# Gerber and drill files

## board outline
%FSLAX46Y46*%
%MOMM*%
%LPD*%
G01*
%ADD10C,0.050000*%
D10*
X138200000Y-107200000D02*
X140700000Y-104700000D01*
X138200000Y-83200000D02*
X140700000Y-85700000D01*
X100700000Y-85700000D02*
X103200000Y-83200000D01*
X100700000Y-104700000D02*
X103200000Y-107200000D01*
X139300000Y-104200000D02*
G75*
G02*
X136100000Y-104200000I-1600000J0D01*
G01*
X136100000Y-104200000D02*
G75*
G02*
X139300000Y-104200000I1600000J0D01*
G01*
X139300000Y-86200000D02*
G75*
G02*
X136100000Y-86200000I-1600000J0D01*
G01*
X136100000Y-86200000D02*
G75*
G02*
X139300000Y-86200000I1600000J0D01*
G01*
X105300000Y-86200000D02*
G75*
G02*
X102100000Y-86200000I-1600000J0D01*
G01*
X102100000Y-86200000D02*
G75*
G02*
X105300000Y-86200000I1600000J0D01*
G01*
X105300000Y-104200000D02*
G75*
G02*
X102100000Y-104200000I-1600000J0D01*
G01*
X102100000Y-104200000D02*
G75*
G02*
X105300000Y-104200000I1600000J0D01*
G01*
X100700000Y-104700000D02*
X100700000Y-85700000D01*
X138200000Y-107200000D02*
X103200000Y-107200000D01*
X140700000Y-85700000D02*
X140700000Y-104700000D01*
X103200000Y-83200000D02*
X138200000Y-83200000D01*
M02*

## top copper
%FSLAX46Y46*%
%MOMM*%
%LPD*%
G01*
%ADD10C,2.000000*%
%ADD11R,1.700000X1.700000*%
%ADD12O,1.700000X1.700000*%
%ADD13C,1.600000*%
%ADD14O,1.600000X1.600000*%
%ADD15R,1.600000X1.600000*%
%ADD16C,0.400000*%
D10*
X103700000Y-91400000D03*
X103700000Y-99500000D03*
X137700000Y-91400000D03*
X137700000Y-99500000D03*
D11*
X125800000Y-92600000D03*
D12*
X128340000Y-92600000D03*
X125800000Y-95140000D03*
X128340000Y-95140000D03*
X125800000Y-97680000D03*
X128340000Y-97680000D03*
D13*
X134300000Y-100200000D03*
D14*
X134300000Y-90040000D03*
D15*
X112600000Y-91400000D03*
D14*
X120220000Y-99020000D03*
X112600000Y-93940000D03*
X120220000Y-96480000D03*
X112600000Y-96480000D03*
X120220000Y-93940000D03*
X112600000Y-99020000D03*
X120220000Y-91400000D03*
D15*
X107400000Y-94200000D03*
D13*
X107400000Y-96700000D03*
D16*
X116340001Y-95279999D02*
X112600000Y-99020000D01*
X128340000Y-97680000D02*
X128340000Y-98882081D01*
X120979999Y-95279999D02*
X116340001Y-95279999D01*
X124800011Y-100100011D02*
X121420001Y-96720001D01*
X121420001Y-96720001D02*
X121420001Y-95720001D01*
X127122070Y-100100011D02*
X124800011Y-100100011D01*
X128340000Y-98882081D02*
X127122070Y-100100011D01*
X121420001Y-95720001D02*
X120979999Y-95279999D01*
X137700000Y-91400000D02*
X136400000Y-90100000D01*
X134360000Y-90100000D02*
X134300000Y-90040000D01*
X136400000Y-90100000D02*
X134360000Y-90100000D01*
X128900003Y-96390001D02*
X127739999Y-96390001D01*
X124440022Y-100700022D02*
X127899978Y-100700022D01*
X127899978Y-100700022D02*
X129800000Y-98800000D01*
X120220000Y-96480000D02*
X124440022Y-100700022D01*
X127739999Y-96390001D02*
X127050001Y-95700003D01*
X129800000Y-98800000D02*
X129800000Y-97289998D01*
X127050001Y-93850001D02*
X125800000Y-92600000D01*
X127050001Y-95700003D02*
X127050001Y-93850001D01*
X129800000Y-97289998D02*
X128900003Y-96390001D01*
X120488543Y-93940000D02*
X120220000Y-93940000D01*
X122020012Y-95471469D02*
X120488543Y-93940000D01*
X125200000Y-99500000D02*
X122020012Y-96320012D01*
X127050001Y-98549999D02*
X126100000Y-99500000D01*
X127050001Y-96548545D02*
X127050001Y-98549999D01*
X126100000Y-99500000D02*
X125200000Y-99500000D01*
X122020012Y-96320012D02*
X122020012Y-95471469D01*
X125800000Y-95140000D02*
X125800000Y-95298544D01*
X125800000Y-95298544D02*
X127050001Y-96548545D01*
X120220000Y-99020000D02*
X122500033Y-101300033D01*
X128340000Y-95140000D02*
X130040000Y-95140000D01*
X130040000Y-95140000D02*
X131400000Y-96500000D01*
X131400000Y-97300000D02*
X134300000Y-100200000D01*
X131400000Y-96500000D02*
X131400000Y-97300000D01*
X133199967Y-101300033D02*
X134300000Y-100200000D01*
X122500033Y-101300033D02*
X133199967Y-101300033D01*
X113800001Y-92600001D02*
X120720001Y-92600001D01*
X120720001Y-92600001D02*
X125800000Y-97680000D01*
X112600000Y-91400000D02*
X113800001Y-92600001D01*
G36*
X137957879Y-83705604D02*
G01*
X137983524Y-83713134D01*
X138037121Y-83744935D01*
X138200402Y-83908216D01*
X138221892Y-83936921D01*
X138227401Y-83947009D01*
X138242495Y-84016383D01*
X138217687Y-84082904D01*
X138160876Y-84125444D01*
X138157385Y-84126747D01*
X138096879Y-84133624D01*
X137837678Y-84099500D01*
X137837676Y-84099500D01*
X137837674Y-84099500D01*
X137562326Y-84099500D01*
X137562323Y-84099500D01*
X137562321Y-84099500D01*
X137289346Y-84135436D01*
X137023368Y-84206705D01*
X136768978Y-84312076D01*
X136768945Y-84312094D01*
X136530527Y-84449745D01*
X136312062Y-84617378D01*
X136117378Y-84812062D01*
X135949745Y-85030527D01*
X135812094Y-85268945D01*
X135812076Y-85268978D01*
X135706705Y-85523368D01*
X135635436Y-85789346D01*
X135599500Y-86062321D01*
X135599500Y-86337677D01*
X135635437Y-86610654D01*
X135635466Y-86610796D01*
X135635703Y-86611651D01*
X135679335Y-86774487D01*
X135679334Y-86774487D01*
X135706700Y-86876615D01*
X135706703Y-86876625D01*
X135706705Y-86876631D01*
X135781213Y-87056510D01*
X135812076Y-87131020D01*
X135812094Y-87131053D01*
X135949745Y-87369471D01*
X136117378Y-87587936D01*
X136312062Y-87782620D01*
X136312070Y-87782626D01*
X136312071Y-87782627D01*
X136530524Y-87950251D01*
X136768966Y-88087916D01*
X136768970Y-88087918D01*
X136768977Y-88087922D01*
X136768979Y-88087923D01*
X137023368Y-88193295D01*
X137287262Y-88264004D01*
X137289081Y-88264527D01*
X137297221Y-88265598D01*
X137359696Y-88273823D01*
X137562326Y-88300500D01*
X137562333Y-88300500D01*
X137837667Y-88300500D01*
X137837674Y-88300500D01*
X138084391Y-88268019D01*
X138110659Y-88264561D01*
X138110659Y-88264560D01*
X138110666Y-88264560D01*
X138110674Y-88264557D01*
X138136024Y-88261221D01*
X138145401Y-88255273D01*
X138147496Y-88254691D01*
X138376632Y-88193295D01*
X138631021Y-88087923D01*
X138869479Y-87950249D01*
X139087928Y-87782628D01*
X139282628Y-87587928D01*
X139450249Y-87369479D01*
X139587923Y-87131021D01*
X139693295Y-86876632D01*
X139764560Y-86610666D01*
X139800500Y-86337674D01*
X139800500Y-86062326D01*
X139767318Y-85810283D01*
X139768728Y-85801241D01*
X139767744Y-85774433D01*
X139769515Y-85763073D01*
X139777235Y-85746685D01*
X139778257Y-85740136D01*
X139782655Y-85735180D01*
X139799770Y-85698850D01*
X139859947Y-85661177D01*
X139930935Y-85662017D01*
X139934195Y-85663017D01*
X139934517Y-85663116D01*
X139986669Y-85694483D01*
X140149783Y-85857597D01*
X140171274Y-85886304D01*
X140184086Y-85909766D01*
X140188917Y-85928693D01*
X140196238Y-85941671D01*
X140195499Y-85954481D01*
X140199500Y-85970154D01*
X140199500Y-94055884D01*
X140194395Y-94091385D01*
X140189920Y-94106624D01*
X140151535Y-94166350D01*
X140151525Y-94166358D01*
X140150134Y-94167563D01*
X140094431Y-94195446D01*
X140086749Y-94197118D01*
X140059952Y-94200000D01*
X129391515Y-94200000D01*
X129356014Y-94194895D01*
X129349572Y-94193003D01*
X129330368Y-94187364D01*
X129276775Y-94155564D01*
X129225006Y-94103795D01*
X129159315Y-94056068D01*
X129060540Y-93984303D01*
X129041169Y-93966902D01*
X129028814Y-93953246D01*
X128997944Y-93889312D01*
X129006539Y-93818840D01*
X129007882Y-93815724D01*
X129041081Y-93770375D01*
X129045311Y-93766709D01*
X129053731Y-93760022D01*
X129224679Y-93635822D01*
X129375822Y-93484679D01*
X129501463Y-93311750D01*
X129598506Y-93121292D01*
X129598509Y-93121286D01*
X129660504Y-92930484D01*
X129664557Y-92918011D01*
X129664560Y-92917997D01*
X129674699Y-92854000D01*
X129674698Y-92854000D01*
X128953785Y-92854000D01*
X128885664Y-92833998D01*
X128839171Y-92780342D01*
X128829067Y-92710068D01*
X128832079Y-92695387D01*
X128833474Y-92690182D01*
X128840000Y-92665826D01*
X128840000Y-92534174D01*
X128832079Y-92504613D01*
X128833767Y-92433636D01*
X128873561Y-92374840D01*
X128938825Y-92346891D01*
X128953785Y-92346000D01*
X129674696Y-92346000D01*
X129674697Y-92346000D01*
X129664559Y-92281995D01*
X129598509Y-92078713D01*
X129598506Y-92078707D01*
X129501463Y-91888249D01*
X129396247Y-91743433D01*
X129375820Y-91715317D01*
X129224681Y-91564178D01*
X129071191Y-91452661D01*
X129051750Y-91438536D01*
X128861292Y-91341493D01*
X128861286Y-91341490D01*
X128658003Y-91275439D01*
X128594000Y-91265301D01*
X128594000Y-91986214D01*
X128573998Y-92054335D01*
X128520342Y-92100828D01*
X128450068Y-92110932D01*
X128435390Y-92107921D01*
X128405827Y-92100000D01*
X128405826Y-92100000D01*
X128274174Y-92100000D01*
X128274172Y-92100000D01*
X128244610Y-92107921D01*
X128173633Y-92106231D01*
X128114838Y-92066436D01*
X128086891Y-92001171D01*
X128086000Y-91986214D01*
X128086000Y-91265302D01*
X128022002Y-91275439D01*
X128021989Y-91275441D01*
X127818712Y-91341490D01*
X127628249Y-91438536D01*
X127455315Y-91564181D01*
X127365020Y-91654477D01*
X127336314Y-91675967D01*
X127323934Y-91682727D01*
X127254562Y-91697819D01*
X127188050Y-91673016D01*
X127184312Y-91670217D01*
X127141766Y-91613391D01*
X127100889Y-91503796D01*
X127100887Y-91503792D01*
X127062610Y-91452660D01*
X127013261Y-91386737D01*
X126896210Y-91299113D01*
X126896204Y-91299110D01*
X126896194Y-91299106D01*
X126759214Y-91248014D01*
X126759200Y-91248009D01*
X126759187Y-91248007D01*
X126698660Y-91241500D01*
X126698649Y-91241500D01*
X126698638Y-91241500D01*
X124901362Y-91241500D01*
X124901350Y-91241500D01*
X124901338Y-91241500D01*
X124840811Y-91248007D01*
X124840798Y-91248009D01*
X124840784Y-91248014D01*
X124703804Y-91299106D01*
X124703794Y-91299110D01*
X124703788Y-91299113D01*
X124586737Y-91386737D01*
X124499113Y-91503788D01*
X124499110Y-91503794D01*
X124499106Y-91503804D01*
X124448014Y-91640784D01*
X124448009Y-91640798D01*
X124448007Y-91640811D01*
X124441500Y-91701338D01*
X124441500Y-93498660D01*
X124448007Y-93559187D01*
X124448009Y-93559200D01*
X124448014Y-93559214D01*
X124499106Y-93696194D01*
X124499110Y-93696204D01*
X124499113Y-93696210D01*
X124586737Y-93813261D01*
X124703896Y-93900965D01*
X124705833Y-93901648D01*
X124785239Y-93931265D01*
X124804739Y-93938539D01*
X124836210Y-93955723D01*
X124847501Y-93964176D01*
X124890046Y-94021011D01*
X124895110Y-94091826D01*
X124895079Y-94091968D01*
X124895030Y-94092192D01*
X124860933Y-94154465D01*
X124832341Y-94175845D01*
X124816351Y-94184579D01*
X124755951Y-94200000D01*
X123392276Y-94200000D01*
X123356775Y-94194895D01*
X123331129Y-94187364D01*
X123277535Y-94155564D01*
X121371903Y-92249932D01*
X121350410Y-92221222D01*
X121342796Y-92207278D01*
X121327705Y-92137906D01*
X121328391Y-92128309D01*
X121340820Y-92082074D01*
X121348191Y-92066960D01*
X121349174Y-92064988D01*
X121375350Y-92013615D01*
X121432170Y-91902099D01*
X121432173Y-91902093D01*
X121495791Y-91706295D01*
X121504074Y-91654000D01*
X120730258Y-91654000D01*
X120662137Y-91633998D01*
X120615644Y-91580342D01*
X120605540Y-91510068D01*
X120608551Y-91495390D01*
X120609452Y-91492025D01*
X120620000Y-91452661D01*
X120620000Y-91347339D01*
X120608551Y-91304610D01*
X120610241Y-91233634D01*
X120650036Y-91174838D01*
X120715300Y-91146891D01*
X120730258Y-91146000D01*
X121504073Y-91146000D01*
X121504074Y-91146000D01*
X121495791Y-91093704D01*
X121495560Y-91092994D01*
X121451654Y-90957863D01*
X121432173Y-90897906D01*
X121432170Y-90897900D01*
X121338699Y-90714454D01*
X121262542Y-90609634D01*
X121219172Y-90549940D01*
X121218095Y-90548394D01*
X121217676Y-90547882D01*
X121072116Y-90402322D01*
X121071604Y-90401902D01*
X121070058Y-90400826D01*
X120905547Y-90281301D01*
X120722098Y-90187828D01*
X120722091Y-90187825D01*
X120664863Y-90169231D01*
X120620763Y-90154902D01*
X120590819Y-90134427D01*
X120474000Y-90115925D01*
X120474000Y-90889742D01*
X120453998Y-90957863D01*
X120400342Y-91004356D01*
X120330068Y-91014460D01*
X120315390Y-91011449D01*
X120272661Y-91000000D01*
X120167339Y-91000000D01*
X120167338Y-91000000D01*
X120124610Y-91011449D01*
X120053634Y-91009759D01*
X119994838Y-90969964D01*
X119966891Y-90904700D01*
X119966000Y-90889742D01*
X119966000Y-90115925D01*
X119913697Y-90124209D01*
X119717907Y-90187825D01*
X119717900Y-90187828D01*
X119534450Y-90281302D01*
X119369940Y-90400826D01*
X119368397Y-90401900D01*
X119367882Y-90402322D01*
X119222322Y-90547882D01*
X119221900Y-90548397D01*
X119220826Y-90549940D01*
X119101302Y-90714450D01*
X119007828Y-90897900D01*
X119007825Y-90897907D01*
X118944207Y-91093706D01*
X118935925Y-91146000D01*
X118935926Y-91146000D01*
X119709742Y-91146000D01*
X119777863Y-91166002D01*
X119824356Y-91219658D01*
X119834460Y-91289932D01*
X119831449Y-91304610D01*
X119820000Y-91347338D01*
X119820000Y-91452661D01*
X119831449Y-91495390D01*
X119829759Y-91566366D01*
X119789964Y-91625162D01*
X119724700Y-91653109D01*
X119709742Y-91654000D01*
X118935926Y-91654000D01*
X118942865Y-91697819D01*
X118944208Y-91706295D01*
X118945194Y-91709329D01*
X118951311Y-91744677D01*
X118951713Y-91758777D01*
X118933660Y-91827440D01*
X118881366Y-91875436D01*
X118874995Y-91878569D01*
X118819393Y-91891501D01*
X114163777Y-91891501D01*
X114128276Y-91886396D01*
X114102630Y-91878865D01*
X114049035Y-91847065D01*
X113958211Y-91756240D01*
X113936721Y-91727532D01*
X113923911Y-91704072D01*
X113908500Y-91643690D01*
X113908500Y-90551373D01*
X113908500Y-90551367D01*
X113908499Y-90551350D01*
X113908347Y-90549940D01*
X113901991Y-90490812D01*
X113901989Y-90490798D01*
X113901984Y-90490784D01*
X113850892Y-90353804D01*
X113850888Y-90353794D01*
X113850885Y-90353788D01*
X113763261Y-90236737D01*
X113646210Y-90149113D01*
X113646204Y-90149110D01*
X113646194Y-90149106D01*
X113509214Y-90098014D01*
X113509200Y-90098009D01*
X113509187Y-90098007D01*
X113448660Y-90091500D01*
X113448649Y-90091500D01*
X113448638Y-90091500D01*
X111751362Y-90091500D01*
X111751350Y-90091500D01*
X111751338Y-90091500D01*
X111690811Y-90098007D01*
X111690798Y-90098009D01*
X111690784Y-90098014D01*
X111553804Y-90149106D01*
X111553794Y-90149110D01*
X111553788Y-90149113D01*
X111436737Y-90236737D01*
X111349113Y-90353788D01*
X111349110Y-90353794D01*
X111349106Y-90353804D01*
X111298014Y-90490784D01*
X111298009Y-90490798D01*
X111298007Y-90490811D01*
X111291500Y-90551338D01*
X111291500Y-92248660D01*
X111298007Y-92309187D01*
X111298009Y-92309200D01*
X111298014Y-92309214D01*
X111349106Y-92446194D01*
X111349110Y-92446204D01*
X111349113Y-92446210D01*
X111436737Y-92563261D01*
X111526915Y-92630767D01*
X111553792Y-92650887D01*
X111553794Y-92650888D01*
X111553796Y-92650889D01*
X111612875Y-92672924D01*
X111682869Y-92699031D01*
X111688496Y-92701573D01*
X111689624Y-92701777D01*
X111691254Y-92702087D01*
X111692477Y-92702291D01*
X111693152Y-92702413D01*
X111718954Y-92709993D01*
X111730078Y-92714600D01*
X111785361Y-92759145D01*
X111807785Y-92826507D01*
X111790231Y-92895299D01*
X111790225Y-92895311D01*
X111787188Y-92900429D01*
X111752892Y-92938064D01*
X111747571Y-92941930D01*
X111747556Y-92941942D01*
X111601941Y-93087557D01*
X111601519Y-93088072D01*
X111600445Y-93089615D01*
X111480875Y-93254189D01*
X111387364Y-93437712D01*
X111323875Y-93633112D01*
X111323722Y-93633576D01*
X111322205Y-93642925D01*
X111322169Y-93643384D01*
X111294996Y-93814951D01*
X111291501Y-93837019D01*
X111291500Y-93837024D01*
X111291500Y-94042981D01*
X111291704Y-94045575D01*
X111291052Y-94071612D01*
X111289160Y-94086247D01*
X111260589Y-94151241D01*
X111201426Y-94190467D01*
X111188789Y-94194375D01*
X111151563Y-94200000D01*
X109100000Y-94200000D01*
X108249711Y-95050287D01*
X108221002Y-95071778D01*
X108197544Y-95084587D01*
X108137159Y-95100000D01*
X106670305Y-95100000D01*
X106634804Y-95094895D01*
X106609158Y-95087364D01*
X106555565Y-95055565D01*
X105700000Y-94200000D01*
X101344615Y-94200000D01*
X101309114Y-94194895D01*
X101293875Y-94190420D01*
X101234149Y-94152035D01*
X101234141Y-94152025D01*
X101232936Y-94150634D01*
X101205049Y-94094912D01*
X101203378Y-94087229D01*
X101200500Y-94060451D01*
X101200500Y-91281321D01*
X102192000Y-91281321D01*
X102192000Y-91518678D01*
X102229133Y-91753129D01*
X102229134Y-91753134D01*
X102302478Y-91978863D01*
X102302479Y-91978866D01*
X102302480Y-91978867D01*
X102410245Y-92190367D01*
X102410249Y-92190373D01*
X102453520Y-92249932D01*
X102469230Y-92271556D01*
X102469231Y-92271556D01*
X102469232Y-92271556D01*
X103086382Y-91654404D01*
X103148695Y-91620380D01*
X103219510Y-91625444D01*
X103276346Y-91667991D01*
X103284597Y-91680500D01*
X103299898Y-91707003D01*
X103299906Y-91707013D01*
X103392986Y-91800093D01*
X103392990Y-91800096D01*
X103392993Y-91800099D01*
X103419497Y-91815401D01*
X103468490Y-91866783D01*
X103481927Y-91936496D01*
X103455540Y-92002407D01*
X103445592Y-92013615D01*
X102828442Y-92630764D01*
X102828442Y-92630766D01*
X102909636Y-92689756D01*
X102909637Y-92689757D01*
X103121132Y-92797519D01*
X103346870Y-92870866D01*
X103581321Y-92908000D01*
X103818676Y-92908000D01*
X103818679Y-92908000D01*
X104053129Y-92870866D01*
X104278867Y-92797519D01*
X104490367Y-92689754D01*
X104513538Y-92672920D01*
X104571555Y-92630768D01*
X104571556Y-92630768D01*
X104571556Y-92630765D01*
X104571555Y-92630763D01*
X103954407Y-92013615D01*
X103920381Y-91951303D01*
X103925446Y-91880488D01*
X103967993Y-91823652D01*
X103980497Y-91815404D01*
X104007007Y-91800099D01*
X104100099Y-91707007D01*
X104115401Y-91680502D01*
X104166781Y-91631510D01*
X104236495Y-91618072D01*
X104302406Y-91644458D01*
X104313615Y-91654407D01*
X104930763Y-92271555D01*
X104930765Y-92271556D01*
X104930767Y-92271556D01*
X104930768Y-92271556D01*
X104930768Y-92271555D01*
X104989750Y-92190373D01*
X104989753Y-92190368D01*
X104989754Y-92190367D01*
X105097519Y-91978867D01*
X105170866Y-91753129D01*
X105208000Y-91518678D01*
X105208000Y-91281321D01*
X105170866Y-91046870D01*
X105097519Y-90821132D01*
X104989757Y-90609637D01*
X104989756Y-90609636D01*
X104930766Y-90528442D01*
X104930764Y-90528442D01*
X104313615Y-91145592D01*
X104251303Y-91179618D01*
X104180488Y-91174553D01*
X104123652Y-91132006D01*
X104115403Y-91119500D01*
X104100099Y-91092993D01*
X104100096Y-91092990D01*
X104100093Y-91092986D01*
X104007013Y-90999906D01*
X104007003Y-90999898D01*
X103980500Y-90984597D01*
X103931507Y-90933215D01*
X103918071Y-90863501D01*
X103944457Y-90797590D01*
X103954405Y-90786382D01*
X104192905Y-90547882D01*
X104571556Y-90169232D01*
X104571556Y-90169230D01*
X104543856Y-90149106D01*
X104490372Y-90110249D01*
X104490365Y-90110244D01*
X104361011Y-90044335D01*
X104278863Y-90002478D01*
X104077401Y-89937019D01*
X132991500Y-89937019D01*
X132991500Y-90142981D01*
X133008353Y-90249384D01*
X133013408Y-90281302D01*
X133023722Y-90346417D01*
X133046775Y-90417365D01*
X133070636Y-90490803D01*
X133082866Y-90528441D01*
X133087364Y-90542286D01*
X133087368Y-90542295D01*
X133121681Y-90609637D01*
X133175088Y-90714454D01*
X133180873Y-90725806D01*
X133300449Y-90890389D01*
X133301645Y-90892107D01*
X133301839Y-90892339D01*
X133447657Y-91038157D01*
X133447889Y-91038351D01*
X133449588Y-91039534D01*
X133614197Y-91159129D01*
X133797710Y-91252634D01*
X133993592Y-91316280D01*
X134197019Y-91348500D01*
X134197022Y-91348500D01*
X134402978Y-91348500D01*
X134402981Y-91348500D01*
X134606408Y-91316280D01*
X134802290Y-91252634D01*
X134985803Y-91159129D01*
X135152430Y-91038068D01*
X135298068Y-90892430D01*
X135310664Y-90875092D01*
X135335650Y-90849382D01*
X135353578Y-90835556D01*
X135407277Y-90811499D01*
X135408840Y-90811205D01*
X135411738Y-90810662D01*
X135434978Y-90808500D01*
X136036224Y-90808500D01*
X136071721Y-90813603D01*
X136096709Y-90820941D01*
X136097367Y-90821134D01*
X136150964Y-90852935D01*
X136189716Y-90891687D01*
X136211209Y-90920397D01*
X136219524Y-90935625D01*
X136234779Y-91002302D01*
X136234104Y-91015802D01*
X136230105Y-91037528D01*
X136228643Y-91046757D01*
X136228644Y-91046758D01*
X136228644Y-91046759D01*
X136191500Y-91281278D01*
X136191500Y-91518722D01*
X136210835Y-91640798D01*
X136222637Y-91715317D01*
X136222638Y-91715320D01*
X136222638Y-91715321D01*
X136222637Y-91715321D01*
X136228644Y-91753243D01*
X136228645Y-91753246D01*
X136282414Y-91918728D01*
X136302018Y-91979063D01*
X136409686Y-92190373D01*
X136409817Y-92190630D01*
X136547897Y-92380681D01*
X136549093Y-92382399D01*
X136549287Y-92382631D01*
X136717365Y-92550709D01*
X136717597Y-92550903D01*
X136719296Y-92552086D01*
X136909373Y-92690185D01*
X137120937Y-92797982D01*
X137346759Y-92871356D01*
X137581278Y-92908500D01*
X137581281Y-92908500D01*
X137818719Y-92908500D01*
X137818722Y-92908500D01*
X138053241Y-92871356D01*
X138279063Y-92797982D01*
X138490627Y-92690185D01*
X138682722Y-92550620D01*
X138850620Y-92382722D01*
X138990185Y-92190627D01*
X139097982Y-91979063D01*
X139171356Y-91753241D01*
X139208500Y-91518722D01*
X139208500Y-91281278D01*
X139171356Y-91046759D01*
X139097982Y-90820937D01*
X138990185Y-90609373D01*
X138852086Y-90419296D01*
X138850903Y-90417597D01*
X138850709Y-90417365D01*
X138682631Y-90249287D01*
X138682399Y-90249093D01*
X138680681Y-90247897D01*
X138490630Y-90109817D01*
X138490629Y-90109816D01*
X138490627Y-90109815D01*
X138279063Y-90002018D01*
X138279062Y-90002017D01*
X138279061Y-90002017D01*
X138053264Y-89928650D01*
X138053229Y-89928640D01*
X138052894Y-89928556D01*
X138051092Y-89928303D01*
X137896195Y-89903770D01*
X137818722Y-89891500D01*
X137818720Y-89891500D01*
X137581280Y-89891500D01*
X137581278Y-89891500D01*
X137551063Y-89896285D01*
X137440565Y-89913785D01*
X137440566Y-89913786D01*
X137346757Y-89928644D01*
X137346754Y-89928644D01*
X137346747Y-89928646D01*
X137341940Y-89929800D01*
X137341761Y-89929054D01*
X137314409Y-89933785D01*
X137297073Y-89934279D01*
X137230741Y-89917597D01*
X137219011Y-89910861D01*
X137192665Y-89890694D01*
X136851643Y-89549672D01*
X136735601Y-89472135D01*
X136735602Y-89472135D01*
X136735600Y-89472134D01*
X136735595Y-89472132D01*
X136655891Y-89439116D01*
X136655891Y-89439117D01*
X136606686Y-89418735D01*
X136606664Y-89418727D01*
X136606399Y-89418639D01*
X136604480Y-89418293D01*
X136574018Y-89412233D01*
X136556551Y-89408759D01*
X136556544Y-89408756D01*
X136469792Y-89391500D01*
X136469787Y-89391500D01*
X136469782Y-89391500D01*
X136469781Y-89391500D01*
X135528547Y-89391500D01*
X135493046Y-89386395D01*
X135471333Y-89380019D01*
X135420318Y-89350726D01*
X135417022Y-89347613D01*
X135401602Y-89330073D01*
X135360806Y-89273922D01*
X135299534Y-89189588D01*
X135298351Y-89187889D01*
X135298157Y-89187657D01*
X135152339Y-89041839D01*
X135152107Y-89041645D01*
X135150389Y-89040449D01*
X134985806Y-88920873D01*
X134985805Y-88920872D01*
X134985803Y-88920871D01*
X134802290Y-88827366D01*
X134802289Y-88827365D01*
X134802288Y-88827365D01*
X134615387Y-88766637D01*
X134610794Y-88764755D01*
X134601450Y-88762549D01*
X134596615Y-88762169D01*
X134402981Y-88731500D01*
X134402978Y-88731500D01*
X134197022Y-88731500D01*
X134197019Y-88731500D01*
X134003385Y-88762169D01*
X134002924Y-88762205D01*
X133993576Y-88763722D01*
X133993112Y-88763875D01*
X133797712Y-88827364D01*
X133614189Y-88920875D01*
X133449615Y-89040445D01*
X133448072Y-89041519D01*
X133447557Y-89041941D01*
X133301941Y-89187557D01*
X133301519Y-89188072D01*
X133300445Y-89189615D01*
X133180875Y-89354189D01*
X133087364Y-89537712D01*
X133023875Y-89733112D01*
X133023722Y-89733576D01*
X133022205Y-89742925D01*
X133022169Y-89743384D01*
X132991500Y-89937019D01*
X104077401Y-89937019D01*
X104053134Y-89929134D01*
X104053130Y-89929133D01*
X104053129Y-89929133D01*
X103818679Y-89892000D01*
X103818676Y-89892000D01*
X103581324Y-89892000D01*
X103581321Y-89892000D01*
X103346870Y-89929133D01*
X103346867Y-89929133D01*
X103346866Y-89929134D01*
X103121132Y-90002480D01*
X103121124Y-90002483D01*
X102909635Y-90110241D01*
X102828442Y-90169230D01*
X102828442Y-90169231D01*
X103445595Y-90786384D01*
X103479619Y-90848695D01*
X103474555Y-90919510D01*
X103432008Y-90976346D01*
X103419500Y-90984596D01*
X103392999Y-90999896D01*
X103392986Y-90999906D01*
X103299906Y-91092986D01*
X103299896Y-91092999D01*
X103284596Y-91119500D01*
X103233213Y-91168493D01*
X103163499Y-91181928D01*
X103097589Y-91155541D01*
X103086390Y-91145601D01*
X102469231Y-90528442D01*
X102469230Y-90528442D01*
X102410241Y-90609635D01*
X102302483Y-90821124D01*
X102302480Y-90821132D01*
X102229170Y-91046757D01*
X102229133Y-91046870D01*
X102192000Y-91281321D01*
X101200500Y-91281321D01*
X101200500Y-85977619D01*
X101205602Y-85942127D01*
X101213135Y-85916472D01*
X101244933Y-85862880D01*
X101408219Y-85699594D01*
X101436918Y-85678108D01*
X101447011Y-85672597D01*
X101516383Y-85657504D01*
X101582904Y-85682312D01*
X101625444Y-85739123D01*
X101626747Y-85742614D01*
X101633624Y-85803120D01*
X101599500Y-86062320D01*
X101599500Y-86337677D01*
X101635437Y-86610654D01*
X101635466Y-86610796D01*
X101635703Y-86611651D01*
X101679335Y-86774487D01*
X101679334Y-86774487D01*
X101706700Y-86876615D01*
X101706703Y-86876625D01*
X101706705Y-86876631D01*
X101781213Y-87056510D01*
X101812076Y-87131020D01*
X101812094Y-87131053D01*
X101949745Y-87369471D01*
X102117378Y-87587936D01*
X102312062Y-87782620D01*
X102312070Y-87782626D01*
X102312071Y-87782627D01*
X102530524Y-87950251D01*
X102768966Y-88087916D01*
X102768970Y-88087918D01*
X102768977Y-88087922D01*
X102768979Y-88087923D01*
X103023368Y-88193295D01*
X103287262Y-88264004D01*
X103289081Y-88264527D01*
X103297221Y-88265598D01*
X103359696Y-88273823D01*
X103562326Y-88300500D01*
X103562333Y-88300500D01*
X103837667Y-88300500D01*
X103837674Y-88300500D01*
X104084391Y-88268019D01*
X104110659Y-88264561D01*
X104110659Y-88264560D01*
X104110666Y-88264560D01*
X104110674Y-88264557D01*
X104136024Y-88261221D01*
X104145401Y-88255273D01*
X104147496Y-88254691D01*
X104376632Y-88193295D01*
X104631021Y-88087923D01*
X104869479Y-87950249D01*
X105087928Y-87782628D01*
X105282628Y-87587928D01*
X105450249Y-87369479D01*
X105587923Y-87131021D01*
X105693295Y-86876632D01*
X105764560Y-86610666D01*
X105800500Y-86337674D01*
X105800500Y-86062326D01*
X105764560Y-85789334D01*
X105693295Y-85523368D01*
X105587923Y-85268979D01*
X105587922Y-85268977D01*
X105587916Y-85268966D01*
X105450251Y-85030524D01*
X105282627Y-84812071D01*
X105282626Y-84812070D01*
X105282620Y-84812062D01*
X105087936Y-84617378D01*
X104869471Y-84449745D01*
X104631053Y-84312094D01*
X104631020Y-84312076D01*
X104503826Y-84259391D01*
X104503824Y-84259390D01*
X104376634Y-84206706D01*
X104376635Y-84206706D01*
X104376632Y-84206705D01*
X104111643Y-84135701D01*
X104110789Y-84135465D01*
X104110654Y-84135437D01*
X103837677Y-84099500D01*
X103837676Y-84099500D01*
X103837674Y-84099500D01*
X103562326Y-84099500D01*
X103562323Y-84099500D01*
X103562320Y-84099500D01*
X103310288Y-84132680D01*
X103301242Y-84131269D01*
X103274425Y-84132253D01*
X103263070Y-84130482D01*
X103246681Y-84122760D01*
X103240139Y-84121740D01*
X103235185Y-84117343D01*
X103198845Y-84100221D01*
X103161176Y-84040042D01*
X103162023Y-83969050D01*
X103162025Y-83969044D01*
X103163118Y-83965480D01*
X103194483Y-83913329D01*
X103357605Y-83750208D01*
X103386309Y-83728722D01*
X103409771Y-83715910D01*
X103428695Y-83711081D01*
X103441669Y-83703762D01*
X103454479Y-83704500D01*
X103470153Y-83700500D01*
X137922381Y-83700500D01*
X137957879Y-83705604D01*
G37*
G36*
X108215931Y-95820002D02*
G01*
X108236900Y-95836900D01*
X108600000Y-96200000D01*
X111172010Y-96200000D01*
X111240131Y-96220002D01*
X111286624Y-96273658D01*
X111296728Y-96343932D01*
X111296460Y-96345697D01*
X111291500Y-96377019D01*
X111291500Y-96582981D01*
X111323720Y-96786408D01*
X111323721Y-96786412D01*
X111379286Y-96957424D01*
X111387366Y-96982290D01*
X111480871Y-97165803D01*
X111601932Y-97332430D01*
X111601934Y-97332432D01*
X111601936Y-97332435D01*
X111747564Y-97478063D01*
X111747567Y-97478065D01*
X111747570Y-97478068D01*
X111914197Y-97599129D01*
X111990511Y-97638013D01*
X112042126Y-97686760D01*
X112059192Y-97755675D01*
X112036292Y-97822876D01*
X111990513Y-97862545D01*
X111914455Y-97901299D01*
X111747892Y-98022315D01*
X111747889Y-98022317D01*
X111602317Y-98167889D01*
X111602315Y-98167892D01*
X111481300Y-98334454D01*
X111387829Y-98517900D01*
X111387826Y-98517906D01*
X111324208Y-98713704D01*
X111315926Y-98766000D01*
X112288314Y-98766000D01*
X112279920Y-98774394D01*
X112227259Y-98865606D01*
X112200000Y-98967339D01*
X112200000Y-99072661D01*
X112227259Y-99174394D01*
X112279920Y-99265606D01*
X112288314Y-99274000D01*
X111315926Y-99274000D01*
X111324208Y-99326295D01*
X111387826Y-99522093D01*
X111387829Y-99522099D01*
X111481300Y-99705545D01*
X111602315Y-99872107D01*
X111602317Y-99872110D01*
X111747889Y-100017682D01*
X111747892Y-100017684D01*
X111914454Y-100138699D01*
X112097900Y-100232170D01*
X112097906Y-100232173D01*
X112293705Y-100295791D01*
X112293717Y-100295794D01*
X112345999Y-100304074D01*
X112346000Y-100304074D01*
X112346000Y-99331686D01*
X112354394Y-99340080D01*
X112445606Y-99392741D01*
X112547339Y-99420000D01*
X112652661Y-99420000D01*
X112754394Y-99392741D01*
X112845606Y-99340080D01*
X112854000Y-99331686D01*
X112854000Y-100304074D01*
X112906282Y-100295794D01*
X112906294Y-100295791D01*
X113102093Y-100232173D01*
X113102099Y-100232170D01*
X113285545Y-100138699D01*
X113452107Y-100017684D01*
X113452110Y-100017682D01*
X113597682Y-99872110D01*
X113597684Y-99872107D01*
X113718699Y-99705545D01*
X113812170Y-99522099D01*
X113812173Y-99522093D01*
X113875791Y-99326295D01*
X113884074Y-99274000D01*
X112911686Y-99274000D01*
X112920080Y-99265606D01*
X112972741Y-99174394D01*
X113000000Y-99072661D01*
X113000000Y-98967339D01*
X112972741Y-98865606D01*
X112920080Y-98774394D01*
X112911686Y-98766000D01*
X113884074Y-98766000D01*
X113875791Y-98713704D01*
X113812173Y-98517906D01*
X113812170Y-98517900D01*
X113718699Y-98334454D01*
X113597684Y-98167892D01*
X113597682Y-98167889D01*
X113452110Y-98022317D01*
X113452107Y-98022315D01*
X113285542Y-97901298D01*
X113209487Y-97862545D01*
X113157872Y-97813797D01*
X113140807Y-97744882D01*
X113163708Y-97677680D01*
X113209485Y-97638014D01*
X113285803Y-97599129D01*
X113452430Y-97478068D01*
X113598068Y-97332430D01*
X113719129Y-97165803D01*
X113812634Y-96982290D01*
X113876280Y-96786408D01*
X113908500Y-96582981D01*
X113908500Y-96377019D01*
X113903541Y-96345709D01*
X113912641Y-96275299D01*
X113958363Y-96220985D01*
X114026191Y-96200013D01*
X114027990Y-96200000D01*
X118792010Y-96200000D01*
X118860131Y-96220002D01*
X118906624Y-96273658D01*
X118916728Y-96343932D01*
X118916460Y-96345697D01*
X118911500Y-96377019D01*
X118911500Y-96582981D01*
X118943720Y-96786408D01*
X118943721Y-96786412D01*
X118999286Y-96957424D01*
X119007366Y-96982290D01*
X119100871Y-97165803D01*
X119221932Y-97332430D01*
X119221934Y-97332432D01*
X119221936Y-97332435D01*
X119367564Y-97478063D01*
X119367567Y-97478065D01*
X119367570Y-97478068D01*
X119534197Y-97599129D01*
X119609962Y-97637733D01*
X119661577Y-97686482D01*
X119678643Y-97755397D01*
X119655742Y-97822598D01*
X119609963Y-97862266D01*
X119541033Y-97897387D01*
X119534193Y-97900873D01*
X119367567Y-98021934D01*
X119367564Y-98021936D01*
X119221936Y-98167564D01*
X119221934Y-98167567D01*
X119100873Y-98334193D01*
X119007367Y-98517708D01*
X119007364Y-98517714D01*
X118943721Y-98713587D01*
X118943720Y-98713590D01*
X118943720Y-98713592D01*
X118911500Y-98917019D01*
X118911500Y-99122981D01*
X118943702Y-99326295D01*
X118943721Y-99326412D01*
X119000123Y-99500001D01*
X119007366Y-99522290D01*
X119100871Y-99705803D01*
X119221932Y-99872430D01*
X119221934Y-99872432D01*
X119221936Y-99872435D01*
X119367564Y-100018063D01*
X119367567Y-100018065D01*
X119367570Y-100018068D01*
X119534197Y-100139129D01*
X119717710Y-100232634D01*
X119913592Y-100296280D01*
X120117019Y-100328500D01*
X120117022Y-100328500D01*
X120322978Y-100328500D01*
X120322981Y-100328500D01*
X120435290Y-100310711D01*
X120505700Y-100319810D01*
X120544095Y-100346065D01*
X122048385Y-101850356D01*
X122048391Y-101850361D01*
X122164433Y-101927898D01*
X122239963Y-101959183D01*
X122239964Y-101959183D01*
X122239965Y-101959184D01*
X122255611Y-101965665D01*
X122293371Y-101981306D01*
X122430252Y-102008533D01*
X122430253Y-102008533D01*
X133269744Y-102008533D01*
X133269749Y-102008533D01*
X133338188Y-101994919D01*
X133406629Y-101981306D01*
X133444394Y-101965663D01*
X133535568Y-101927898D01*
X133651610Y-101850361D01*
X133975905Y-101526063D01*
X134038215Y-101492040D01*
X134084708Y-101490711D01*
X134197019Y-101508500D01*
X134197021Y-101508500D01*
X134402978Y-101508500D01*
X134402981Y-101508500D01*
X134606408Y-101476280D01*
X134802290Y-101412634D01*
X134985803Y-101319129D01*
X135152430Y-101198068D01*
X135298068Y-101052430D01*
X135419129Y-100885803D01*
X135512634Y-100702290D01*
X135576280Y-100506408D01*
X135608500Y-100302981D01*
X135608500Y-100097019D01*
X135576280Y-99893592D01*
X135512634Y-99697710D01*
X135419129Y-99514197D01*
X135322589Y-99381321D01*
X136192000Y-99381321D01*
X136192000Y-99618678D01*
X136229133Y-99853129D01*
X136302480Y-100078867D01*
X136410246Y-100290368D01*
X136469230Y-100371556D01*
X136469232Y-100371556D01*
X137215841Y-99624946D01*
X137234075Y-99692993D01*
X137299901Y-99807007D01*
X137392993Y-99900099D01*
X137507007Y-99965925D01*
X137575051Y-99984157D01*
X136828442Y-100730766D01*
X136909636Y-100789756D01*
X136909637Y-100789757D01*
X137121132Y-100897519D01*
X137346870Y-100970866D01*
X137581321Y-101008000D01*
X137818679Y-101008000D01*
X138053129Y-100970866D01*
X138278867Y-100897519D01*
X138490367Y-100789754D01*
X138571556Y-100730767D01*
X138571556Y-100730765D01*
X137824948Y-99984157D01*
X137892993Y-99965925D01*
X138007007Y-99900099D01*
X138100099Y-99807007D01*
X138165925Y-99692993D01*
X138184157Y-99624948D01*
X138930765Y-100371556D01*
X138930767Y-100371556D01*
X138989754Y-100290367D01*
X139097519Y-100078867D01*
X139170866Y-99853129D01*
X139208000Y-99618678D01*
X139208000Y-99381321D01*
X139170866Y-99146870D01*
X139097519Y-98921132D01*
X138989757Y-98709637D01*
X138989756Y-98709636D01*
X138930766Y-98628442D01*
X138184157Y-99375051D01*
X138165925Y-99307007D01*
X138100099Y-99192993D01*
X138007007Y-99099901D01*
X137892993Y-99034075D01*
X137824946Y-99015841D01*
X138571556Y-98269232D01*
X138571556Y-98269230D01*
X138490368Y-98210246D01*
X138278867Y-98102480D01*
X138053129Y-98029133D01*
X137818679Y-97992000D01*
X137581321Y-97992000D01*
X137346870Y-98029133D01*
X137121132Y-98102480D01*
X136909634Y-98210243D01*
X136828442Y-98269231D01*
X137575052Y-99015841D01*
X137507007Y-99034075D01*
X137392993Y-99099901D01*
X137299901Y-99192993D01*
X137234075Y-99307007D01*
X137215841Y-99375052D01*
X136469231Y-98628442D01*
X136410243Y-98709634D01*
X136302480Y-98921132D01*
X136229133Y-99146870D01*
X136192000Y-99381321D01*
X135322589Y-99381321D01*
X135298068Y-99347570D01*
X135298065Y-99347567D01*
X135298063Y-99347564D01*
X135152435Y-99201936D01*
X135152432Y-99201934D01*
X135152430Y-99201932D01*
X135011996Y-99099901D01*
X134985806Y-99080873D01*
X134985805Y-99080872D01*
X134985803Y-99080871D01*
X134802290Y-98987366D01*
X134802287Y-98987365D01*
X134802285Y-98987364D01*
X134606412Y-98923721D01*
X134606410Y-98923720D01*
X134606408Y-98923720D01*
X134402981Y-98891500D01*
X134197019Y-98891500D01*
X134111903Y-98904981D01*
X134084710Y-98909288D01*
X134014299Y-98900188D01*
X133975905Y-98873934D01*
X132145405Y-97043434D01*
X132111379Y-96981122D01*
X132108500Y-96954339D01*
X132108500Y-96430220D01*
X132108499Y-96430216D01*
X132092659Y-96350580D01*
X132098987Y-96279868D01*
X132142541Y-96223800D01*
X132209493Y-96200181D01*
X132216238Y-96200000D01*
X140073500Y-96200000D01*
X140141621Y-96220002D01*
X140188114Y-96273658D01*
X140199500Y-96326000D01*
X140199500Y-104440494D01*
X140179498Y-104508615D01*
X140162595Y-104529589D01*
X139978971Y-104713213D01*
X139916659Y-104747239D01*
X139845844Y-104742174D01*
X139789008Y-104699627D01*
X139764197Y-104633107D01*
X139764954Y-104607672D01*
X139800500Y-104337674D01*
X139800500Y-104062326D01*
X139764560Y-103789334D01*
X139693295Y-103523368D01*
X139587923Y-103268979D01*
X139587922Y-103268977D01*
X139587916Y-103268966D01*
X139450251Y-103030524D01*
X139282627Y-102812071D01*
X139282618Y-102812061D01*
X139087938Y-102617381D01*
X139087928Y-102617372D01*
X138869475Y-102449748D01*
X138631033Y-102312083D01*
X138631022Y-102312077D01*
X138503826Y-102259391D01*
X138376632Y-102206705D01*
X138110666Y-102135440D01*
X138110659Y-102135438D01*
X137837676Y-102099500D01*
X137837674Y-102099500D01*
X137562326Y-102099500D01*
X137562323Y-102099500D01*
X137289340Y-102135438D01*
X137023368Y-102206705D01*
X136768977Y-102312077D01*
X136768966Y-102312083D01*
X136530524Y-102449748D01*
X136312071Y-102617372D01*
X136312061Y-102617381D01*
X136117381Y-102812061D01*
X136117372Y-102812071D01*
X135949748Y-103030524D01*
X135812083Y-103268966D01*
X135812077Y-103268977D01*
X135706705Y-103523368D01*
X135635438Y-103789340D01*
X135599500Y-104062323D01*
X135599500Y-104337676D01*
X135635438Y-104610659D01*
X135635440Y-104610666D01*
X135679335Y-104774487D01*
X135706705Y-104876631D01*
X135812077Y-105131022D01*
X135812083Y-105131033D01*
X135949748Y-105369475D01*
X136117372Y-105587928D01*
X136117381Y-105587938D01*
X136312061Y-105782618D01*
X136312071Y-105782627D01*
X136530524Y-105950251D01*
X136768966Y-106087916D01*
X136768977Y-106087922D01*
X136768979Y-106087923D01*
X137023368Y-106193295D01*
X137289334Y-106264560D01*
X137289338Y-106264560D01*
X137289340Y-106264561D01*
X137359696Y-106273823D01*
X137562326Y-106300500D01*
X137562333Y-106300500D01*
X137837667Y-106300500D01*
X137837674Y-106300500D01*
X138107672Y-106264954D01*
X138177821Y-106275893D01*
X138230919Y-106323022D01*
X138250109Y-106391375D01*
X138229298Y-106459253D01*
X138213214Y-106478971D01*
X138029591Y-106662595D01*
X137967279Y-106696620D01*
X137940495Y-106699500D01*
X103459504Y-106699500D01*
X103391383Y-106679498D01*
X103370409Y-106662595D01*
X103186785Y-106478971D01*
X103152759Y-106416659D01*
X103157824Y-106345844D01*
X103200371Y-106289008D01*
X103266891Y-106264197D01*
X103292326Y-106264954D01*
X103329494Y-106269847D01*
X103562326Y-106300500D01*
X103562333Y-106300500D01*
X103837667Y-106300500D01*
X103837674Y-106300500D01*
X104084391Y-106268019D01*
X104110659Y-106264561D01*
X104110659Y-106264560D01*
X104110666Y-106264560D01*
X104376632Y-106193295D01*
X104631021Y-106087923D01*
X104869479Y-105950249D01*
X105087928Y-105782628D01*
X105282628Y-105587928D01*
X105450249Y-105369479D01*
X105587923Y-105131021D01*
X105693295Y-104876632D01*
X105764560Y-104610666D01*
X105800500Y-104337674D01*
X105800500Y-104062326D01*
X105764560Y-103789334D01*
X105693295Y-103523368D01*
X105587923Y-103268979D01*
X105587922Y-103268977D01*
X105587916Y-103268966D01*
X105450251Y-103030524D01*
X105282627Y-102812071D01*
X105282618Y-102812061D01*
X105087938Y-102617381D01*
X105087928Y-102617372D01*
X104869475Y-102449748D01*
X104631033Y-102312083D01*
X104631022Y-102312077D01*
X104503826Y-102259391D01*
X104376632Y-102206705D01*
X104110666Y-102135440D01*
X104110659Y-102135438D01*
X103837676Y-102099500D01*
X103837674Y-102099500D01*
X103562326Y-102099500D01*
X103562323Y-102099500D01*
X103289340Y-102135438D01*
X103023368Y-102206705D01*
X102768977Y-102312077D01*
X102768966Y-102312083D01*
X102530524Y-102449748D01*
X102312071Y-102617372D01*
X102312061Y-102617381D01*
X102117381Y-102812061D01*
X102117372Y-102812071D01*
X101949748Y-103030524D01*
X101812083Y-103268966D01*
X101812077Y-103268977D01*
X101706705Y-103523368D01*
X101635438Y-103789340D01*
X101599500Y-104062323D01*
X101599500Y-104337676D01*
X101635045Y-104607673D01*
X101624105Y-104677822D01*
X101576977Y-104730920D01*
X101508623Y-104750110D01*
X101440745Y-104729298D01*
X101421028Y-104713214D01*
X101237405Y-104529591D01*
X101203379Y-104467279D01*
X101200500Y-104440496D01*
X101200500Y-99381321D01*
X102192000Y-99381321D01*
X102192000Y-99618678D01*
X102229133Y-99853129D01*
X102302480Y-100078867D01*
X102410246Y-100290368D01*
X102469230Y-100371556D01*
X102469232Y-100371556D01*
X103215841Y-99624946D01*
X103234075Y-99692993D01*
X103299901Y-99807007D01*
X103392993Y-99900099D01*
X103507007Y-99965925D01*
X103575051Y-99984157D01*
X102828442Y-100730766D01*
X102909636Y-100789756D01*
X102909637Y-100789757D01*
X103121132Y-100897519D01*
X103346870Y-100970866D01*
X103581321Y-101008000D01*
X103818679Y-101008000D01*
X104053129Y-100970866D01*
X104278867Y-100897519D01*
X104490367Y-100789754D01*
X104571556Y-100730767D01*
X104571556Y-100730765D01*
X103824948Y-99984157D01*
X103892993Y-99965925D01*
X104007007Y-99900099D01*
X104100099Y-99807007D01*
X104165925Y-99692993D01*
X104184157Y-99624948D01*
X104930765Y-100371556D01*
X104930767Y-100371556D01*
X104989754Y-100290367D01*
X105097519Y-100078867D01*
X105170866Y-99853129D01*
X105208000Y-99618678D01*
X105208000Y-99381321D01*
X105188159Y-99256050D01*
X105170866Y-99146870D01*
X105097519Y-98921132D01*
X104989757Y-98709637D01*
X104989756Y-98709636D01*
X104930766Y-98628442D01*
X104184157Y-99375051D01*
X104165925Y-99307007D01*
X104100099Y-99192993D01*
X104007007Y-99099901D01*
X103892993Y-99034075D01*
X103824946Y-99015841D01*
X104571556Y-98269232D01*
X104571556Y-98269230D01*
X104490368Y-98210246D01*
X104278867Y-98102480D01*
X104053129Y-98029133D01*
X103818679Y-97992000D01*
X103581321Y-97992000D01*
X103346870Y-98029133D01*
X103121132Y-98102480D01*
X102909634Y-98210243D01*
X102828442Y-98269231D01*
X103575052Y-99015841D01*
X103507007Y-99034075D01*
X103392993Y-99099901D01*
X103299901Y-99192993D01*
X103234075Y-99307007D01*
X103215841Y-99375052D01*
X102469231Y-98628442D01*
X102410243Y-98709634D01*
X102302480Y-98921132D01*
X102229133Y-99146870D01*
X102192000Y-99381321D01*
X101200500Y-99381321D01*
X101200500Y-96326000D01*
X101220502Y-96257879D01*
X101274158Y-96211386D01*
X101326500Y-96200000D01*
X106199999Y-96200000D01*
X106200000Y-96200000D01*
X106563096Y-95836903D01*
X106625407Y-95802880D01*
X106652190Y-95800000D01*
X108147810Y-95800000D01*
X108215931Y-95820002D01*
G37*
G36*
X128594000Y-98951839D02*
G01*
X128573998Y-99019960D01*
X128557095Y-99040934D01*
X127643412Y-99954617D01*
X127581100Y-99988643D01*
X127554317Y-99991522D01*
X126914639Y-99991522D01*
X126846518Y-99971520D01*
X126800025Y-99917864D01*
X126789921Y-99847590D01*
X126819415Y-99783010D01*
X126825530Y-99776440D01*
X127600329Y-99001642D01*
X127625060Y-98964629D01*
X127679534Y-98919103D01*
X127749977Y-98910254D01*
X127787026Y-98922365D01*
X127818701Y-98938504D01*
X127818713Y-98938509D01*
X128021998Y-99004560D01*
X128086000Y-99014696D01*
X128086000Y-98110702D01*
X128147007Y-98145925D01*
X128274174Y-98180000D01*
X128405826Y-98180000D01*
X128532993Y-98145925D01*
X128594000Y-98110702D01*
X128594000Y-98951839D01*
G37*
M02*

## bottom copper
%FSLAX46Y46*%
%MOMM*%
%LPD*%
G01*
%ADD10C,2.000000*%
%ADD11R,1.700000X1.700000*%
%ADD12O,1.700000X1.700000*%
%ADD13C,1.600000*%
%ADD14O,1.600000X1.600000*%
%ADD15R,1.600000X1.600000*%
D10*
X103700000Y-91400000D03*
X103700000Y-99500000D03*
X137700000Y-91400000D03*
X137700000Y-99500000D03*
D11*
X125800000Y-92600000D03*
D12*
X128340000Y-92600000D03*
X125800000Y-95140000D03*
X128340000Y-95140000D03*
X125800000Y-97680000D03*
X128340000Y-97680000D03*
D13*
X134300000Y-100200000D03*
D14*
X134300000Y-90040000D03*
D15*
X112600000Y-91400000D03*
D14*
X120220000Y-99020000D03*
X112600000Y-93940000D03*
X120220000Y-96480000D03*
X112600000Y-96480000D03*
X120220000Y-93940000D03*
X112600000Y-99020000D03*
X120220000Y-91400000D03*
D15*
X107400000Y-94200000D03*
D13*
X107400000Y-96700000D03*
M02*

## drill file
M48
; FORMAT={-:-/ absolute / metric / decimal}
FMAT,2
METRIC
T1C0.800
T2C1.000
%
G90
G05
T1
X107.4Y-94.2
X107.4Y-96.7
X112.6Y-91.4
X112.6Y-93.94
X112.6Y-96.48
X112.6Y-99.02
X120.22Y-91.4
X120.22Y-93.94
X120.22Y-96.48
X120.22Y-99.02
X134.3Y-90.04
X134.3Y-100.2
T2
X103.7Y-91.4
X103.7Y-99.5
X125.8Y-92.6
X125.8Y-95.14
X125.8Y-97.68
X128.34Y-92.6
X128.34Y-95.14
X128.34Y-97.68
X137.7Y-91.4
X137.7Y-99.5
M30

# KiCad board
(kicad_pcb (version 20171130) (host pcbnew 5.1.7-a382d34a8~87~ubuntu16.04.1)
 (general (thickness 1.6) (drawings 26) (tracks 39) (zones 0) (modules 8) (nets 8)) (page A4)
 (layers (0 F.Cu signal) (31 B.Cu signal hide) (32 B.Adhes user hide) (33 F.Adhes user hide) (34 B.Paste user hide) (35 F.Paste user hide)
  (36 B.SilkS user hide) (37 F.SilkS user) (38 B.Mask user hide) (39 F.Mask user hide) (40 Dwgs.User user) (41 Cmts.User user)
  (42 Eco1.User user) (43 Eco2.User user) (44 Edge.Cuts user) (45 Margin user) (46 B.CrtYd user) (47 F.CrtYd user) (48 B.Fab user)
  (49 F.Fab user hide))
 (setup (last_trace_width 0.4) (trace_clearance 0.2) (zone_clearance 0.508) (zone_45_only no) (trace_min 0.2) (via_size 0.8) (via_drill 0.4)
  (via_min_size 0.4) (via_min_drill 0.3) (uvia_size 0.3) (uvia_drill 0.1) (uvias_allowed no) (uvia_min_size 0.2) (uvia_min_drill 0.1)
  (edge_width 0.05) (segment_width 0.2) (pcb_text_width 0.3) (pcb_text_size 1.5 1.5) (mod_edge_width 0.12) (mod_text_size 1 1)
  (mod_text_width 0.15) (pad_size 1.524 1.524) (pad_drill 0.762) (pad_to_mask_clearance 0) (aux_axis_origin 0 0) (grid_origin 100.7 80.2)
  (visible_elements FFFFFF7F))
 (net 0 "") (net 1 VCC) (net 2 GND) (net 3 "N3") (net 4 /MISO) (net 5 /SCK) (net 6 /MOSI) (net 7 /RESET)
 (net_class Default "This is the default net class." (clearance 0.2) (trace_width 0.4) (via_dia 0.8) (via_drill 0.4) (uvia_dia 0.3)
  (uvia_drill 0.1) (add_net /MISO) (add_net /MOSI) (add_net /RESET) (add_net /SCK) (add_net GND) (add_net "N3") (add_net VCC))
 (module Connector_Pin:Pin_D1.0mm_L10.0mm (layer F.Cu) (at 103.7 91.4)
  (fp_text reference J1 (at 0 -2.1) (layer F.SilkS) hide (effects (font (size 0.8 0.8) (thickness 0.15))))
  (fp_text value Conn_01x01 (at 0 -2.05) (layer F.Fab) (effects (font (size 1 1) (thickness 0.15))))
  (pad 1 thru_hole circle (at 0 0) (size 2 2) (drill 1) (layers *.Cu *.Mask) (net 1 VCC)))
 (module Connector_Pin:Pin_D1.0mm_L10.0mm (layer F.Cu) (at 103.7 99.5)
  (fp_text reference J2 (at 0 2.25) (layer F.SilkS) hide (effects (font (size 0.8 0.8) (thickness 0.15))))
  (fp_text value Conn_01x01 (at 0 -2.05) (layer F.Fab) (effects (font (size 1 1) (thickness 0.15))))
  (pad 1 thru_hole circle (at 0 0) (size 2 2) (drill 1) (layers *.Cu *.Mask) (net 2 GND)))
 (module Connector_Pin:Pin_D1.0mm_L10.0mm (layer F.Cu) (at 137.7 91.4)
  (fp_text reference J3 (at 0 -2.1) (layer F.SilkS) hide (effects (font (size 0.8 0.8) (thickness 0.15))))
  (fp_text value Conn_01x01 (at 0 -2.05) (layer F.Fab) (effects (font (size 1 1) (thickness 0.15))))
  (pad 1 thru_hole circle (at 0 0) (size 2 2) (drill 1) (layers *.Cu *.Mask) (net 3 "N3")))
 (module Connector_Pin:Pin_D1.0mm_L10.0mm (layer F.Cu) (at 137.7 99.5)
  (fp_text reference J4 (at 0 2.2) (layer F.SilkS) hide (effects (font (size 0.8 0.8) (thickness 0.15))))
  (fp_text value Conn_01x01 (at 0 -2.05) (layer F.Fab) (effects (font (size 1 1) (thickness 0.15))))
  (pad 1 thru_hole circle (at 0 0) (size 2 2) (drill 1) (layers *.Cu *.Mask) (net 2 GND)))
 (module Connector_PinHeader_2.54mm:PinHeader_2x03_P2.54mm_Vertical (layer F.Cu) (at 125.8 92.6)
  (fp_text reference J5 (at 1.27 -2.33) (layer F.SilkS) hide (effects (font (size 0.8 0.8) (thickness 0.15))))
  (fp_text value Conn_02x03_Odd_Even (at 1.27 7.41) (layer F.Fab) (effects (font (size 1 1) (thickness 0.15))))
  (pad 1 thru_hole rect (at 0 0) (size 1.7 1.7) (drill 1) (layers *.Cu *.Mask) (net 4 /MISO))
  (pad 2 thru_hole oval (at 2.54 0) (size 1.7 1.7) (drill 1) (layers *.Cu *.Mask) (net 1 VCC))
  (pad 3 thru_hole oval (at 0 2.54) (size 1.7 1.7) (drill 1) (layers *.Cu *.Mask) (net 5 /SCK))
  (pad 4 thru_hole oval (at 2.54 2.54) (size 1.7 1.7) (drill 1) (layers *.Cu *.Mask) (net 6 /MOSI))
  (pad 5 thru_hole oval (at 0 5.08) (size 1.7 1.7) (drill 1) (layers *.Cu *.Mask) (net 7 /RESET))
  (pad 6 thru_hole oval (at 2.54 5.08) (size 1.7 1.7) (drill 1) (layers *.Cu *.Mask) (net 2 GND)))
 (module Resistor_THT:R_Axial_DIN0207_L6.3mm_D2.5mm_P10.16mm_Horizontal (layer F.Cu) (at 134.3 100.2 90)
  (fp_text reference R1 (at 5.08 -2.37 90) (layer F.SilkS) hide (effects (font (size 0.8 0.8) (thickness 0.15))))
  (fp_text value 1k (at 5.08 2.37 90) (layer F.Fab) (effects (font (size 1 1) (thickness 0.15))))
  (pad 1 thru_hole circle (at 0 0 90) (size 1.6 1.6) (drill 0.8) (layers *.Cu *.Mask) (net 6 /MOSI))
  (pad 2 thru_hole oval (at 10.16 0 90) (size 1.6 1.6) (drill 0.8) (layers *.Cu *.Mask) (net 3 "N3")))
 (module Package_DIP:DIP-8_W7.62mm (layer F.Cu) (at 112.6 91.4)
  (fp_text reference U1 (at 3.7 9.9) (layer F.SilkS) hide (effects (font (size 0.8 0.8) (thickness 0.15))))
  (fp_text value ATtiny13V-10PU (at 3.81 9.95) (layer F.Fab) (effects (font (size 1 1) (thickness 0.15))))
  (pad 1 thru_hole rect (at 0 0) (size 1.6 1.6) (drill 0.8) (layers *.Cu *.Mask) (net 7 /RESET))
  (pad 5 thru_hole oval (at 7.62 7.62) (size 1.6 1.6) (drill 0.8) (layers *.Cu *.Mask) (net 6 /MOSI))
  (pad 2 thru_hole oval (at 0 2.54) (size 1.6 1.6) (drill 0.8) (layers *.Cu *.Mask))
  (pad 6 thru_hole oval (at 7.62 5.08) (size 1.6 1.6) (drill 0.8) (layers *.Cu *.Mask) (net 4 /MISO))
  (pad 3 thru_hole oval (at 0 5.08) (size 1.6 1.6) (drill 0.8) (layers *.Cu *.Mask))
  (pad 7 thru_hole oval (at 7.62 2.54) (size 1.6 1.6) (drill 0.8) (layers *.Cu *.Mask) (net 5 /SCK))
  (pad 4 thru_hole oval (at 0 7.62) (size 1.6 1.6) (drill 0.8) (layers *.Cu *.Mask) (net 2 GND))
  (pad 8 thru_hole oval (at 7.62 0) (size 1.6 1.6) (drill 0.8) (layers *.Cu *.Mask) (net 1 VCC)))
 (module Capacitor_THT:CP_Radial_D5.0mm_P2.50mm (layer F.Cu) (at 107.4 94.2 270) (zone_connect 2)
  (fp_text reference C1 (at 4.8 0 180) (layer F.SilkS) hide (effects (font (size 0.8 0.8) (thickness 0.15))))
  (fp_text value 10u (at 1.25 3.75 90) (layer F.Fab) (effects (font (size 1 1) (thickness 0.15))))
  (pad 1 thru_hole rect (at 0 0 270) (size 1.6 1.6) (drill 0.8) (layers *.Cu *.Mask) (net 1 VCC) (zone_connect 2))
  (pad 2 thru_hole circle (at 2.5 0 270) (size 1.6 1.6) (drill 0.8) (layers *.Cu *.Mask) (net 2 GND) (zone_connect 2)))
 (gr_line (start 138.2 107.2) (end 140.7 104.7) (layer Edge.Cuts) (width 0.05))
 (gr_line (start 138.2 83.2) (end 140.7 85.7) (layer Edge.Cuts) (width 0.05))
 (gr_line (start 100.7 85.7) (end 103.2 83.2) (layer Edge.Cuts) (width 0.05))
 (gr_line (start 100.7 104.7) (end 103.2 107.2) (layer Edge.Cuts) (width 0.05))
 (gr_circle (center 137.7 104.2) (end 139.3 104.2) (layer Edge.Cuts) (width 0.05))
 (gr_circle (center 137.7 86.2) (end 139.3 86.2) (layer Edge.Cuts) (width 0.05))
 (gr_circle (center 103.7 86.2) (end 105.3 86.2) (layer Edge.Cuts) (width 0.05))
 (gr_circle (center 103.7 104.2) (end 105.3 104.2) (layer Edge.Cuts) (width 0.05))
 (gr_line (start 100.7 104.7) (end 100.7 85.7) (layer Edge.Cuts) (width 0.05))
 (gr_line (start 138.2 107.2) (end 103.2 107.2) (layer Edge.Cuts) (width 0.05))
 (gr_line (start 140.7 85.7) (end 140.7 104.7) (layer Edge.Cuts) (width 0.05))
 (gr_line (start 103.2 83.2) (end 138.2 83.2) (layer Edge.Cuts) (width 0.05))
 (segment (start 116.340001 95.279999) (end 112.6 99.02) (width 0.4) (layer F.Cu) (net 2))
 (segment (start 128.34 97.68) (end 128.34 98.882081) (width 0.4) (layer F.Cu) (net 2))
 (segment (start 120.979999 95.279999) (end 116.340001 95.279999) (width 0.4) (layer F.Cu) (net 2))
 (segment (start 124.800011 100.100011) (end 121.420001 96.720001) (width 0.4) (layer F.Cu) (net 2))
 (segment (start 121.420001 96.720001) (end 121.420001 95.720001) (width 0.4) (layer F.Cu) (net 2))
 (segment (start 127.12207 100.100011) (end 124.800011 100.100011) (width 0.4) (layer F.Cu) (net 2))
 (segment (start 128.34 98.882081) (end 127.12207 100.100011) (width 0.4) (layer F.Cu) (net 2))
 (segment (start 121.420001 95.720001) (end 120.979999 95.279999) (width 0.4) (layer F.Cu) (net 2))
 (segment (start 137.7 91.4) (end 136.4 90.1) (width 0.4) (layer F.Cu) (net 3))
 (segment (start 134.36 90.1) (end 134.3 90.04) (width 0.4) (layer F.Cu) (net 3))
 (segment (start 136.4 90.1) (end 134.36 90.1) (width 0.4) (layer F.Cu) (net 3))
 (segment (start 128.900003 96.390001) (end 127.739999 96.390001) (width 0.4) (layer F.Cu) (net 4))
 (segment (start 124.440022 100.700022) (end 127.899978 100.700022) (width 0.4) (layer F.Cu) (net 4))
 (segment (start 127.899978 100.700022) (end 129.8 98.8) (width 0.4) (layer F.Cu) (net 4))
 (segment (start 120.22 96.48) (end 124.440022 100.700022) (width 0.4) (layer F.Cu) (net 4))
 (segment (start 127.739999 96.390001) (end 127.050001 95.700003) (width 0.4) (layer F.Cu) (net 4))
 (segment (start 129.8 98.8) (end 129.8 97.289998) (width 0.4) (layer F.Cu) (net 4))
 (segment (start 127.050001 93.850001) (end 125.8 92.6) (width 0.4) (layer F.Cu) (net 4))
 (segment (start 127.050001 95.700003) (end 127.050001 93.850001) (width 0.4) (layer F.Cu) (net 4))
 (segment (start 129.8 97.289998) (end 128.900003 96.390001) (width 0.4) (layer F.Cu) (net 4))
 (segment (start 120.488543 93.94) (end 120.22 93.94) (width 0.4) (layer F.Cu) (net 5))
 (segment (start 122.020012 95.471469) (end 120.488543 93.94) (width 0.4) (layer F.Cu) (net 5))
 (segment (start 125.2 99.5) (end 122.020012 96.320012) (width 0.4) (layer F.Cu) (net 5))
 (segment (start 127.050001 98.549999) (end 126.1 99.5) (width 0.4) (layer F.Cu) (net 5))
 (segment (start 127.050001 96.548545) (end 127.050001 98.549999) (width 0.4) (layer F.Cu) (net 5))
 (segment (start 126.1 99.5) (end 125.2 99.5) (width 0.4) (layer F.Cu) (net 5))
 (segment (start 122.020012 96.320012) (end 122.020012 95.471469) (width 0.4) (layer F.Cu) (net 5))
 (segment (start 125.8 95.14) (end 125.8 95.298544) (width 0.4) (layer F.Cu) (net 5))
 (segment (start 125.8 95.298544) (end 127.050001 96.548545) (width 0.4) (layer F.Cu) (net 5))
 (segment (start 120.22 99.02) (end 122.500033 101.300033) (width 0.4) (layer F.Cu) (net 6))
 (segment (start 128.34 95.14) (end 130.04 95.14) (width 0.4) (layer F.Cu) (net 6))
 (segment (start 130.04 95.14) (end 131.4 96.5) (width 0.4) (layer F.Cu) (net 6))
 (segment (start 131.4 97.3) (end 134.3 100.2) (width 0.4) (layer F.Cu) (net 6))
 (segment (start 131.4 96.5) (end 131.4 97.3) (width 0.4) (layer F.Cu) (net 6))
 (segment (start 133.199967 101.300033) (end 134.3 100.2) (width 0.4) (layer F.Cu) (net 6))
 (segment (start 122.500033 101.300033) (end 133.199967 101.300033) (width 0.4) (layer F.Cu) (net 6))
 (segment (start 113.800001 92.600001) (end 120.720001 92.600001) (width 0.4) (layer F.Cu) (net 7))
 (segment (start 120.720001 92.600001) (end 125.8 97.68) (width 0.4) (layer F.Cu) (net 7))
 (segment (start 112.6 91.4) (end 113.800001 92.600001) (width 0.4) (layer F.Cu) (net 7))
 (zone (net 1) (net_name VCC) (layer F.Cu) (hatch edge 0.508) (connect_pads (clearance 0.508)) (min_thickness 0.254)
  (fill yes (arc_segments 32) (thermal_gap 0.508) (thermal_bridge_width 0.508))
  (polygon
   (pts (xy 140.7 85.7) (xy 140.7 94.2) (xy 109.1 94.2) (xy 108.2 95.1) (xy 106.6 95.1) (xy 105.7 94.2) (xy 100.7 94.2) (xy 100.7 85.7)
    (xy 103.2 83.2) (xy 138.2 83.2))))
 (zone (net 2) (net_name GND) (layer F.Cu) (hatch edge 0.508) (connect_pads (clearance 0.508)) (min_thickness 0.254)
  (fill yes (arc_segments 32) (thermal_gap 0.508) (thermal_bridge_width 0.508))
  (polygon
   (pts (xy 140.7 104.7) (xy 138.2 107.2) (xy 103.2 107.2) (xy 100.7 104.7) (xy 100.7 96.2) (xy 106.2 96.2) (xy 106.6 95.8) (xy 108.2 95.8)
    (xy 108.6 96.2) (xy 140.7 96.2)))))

